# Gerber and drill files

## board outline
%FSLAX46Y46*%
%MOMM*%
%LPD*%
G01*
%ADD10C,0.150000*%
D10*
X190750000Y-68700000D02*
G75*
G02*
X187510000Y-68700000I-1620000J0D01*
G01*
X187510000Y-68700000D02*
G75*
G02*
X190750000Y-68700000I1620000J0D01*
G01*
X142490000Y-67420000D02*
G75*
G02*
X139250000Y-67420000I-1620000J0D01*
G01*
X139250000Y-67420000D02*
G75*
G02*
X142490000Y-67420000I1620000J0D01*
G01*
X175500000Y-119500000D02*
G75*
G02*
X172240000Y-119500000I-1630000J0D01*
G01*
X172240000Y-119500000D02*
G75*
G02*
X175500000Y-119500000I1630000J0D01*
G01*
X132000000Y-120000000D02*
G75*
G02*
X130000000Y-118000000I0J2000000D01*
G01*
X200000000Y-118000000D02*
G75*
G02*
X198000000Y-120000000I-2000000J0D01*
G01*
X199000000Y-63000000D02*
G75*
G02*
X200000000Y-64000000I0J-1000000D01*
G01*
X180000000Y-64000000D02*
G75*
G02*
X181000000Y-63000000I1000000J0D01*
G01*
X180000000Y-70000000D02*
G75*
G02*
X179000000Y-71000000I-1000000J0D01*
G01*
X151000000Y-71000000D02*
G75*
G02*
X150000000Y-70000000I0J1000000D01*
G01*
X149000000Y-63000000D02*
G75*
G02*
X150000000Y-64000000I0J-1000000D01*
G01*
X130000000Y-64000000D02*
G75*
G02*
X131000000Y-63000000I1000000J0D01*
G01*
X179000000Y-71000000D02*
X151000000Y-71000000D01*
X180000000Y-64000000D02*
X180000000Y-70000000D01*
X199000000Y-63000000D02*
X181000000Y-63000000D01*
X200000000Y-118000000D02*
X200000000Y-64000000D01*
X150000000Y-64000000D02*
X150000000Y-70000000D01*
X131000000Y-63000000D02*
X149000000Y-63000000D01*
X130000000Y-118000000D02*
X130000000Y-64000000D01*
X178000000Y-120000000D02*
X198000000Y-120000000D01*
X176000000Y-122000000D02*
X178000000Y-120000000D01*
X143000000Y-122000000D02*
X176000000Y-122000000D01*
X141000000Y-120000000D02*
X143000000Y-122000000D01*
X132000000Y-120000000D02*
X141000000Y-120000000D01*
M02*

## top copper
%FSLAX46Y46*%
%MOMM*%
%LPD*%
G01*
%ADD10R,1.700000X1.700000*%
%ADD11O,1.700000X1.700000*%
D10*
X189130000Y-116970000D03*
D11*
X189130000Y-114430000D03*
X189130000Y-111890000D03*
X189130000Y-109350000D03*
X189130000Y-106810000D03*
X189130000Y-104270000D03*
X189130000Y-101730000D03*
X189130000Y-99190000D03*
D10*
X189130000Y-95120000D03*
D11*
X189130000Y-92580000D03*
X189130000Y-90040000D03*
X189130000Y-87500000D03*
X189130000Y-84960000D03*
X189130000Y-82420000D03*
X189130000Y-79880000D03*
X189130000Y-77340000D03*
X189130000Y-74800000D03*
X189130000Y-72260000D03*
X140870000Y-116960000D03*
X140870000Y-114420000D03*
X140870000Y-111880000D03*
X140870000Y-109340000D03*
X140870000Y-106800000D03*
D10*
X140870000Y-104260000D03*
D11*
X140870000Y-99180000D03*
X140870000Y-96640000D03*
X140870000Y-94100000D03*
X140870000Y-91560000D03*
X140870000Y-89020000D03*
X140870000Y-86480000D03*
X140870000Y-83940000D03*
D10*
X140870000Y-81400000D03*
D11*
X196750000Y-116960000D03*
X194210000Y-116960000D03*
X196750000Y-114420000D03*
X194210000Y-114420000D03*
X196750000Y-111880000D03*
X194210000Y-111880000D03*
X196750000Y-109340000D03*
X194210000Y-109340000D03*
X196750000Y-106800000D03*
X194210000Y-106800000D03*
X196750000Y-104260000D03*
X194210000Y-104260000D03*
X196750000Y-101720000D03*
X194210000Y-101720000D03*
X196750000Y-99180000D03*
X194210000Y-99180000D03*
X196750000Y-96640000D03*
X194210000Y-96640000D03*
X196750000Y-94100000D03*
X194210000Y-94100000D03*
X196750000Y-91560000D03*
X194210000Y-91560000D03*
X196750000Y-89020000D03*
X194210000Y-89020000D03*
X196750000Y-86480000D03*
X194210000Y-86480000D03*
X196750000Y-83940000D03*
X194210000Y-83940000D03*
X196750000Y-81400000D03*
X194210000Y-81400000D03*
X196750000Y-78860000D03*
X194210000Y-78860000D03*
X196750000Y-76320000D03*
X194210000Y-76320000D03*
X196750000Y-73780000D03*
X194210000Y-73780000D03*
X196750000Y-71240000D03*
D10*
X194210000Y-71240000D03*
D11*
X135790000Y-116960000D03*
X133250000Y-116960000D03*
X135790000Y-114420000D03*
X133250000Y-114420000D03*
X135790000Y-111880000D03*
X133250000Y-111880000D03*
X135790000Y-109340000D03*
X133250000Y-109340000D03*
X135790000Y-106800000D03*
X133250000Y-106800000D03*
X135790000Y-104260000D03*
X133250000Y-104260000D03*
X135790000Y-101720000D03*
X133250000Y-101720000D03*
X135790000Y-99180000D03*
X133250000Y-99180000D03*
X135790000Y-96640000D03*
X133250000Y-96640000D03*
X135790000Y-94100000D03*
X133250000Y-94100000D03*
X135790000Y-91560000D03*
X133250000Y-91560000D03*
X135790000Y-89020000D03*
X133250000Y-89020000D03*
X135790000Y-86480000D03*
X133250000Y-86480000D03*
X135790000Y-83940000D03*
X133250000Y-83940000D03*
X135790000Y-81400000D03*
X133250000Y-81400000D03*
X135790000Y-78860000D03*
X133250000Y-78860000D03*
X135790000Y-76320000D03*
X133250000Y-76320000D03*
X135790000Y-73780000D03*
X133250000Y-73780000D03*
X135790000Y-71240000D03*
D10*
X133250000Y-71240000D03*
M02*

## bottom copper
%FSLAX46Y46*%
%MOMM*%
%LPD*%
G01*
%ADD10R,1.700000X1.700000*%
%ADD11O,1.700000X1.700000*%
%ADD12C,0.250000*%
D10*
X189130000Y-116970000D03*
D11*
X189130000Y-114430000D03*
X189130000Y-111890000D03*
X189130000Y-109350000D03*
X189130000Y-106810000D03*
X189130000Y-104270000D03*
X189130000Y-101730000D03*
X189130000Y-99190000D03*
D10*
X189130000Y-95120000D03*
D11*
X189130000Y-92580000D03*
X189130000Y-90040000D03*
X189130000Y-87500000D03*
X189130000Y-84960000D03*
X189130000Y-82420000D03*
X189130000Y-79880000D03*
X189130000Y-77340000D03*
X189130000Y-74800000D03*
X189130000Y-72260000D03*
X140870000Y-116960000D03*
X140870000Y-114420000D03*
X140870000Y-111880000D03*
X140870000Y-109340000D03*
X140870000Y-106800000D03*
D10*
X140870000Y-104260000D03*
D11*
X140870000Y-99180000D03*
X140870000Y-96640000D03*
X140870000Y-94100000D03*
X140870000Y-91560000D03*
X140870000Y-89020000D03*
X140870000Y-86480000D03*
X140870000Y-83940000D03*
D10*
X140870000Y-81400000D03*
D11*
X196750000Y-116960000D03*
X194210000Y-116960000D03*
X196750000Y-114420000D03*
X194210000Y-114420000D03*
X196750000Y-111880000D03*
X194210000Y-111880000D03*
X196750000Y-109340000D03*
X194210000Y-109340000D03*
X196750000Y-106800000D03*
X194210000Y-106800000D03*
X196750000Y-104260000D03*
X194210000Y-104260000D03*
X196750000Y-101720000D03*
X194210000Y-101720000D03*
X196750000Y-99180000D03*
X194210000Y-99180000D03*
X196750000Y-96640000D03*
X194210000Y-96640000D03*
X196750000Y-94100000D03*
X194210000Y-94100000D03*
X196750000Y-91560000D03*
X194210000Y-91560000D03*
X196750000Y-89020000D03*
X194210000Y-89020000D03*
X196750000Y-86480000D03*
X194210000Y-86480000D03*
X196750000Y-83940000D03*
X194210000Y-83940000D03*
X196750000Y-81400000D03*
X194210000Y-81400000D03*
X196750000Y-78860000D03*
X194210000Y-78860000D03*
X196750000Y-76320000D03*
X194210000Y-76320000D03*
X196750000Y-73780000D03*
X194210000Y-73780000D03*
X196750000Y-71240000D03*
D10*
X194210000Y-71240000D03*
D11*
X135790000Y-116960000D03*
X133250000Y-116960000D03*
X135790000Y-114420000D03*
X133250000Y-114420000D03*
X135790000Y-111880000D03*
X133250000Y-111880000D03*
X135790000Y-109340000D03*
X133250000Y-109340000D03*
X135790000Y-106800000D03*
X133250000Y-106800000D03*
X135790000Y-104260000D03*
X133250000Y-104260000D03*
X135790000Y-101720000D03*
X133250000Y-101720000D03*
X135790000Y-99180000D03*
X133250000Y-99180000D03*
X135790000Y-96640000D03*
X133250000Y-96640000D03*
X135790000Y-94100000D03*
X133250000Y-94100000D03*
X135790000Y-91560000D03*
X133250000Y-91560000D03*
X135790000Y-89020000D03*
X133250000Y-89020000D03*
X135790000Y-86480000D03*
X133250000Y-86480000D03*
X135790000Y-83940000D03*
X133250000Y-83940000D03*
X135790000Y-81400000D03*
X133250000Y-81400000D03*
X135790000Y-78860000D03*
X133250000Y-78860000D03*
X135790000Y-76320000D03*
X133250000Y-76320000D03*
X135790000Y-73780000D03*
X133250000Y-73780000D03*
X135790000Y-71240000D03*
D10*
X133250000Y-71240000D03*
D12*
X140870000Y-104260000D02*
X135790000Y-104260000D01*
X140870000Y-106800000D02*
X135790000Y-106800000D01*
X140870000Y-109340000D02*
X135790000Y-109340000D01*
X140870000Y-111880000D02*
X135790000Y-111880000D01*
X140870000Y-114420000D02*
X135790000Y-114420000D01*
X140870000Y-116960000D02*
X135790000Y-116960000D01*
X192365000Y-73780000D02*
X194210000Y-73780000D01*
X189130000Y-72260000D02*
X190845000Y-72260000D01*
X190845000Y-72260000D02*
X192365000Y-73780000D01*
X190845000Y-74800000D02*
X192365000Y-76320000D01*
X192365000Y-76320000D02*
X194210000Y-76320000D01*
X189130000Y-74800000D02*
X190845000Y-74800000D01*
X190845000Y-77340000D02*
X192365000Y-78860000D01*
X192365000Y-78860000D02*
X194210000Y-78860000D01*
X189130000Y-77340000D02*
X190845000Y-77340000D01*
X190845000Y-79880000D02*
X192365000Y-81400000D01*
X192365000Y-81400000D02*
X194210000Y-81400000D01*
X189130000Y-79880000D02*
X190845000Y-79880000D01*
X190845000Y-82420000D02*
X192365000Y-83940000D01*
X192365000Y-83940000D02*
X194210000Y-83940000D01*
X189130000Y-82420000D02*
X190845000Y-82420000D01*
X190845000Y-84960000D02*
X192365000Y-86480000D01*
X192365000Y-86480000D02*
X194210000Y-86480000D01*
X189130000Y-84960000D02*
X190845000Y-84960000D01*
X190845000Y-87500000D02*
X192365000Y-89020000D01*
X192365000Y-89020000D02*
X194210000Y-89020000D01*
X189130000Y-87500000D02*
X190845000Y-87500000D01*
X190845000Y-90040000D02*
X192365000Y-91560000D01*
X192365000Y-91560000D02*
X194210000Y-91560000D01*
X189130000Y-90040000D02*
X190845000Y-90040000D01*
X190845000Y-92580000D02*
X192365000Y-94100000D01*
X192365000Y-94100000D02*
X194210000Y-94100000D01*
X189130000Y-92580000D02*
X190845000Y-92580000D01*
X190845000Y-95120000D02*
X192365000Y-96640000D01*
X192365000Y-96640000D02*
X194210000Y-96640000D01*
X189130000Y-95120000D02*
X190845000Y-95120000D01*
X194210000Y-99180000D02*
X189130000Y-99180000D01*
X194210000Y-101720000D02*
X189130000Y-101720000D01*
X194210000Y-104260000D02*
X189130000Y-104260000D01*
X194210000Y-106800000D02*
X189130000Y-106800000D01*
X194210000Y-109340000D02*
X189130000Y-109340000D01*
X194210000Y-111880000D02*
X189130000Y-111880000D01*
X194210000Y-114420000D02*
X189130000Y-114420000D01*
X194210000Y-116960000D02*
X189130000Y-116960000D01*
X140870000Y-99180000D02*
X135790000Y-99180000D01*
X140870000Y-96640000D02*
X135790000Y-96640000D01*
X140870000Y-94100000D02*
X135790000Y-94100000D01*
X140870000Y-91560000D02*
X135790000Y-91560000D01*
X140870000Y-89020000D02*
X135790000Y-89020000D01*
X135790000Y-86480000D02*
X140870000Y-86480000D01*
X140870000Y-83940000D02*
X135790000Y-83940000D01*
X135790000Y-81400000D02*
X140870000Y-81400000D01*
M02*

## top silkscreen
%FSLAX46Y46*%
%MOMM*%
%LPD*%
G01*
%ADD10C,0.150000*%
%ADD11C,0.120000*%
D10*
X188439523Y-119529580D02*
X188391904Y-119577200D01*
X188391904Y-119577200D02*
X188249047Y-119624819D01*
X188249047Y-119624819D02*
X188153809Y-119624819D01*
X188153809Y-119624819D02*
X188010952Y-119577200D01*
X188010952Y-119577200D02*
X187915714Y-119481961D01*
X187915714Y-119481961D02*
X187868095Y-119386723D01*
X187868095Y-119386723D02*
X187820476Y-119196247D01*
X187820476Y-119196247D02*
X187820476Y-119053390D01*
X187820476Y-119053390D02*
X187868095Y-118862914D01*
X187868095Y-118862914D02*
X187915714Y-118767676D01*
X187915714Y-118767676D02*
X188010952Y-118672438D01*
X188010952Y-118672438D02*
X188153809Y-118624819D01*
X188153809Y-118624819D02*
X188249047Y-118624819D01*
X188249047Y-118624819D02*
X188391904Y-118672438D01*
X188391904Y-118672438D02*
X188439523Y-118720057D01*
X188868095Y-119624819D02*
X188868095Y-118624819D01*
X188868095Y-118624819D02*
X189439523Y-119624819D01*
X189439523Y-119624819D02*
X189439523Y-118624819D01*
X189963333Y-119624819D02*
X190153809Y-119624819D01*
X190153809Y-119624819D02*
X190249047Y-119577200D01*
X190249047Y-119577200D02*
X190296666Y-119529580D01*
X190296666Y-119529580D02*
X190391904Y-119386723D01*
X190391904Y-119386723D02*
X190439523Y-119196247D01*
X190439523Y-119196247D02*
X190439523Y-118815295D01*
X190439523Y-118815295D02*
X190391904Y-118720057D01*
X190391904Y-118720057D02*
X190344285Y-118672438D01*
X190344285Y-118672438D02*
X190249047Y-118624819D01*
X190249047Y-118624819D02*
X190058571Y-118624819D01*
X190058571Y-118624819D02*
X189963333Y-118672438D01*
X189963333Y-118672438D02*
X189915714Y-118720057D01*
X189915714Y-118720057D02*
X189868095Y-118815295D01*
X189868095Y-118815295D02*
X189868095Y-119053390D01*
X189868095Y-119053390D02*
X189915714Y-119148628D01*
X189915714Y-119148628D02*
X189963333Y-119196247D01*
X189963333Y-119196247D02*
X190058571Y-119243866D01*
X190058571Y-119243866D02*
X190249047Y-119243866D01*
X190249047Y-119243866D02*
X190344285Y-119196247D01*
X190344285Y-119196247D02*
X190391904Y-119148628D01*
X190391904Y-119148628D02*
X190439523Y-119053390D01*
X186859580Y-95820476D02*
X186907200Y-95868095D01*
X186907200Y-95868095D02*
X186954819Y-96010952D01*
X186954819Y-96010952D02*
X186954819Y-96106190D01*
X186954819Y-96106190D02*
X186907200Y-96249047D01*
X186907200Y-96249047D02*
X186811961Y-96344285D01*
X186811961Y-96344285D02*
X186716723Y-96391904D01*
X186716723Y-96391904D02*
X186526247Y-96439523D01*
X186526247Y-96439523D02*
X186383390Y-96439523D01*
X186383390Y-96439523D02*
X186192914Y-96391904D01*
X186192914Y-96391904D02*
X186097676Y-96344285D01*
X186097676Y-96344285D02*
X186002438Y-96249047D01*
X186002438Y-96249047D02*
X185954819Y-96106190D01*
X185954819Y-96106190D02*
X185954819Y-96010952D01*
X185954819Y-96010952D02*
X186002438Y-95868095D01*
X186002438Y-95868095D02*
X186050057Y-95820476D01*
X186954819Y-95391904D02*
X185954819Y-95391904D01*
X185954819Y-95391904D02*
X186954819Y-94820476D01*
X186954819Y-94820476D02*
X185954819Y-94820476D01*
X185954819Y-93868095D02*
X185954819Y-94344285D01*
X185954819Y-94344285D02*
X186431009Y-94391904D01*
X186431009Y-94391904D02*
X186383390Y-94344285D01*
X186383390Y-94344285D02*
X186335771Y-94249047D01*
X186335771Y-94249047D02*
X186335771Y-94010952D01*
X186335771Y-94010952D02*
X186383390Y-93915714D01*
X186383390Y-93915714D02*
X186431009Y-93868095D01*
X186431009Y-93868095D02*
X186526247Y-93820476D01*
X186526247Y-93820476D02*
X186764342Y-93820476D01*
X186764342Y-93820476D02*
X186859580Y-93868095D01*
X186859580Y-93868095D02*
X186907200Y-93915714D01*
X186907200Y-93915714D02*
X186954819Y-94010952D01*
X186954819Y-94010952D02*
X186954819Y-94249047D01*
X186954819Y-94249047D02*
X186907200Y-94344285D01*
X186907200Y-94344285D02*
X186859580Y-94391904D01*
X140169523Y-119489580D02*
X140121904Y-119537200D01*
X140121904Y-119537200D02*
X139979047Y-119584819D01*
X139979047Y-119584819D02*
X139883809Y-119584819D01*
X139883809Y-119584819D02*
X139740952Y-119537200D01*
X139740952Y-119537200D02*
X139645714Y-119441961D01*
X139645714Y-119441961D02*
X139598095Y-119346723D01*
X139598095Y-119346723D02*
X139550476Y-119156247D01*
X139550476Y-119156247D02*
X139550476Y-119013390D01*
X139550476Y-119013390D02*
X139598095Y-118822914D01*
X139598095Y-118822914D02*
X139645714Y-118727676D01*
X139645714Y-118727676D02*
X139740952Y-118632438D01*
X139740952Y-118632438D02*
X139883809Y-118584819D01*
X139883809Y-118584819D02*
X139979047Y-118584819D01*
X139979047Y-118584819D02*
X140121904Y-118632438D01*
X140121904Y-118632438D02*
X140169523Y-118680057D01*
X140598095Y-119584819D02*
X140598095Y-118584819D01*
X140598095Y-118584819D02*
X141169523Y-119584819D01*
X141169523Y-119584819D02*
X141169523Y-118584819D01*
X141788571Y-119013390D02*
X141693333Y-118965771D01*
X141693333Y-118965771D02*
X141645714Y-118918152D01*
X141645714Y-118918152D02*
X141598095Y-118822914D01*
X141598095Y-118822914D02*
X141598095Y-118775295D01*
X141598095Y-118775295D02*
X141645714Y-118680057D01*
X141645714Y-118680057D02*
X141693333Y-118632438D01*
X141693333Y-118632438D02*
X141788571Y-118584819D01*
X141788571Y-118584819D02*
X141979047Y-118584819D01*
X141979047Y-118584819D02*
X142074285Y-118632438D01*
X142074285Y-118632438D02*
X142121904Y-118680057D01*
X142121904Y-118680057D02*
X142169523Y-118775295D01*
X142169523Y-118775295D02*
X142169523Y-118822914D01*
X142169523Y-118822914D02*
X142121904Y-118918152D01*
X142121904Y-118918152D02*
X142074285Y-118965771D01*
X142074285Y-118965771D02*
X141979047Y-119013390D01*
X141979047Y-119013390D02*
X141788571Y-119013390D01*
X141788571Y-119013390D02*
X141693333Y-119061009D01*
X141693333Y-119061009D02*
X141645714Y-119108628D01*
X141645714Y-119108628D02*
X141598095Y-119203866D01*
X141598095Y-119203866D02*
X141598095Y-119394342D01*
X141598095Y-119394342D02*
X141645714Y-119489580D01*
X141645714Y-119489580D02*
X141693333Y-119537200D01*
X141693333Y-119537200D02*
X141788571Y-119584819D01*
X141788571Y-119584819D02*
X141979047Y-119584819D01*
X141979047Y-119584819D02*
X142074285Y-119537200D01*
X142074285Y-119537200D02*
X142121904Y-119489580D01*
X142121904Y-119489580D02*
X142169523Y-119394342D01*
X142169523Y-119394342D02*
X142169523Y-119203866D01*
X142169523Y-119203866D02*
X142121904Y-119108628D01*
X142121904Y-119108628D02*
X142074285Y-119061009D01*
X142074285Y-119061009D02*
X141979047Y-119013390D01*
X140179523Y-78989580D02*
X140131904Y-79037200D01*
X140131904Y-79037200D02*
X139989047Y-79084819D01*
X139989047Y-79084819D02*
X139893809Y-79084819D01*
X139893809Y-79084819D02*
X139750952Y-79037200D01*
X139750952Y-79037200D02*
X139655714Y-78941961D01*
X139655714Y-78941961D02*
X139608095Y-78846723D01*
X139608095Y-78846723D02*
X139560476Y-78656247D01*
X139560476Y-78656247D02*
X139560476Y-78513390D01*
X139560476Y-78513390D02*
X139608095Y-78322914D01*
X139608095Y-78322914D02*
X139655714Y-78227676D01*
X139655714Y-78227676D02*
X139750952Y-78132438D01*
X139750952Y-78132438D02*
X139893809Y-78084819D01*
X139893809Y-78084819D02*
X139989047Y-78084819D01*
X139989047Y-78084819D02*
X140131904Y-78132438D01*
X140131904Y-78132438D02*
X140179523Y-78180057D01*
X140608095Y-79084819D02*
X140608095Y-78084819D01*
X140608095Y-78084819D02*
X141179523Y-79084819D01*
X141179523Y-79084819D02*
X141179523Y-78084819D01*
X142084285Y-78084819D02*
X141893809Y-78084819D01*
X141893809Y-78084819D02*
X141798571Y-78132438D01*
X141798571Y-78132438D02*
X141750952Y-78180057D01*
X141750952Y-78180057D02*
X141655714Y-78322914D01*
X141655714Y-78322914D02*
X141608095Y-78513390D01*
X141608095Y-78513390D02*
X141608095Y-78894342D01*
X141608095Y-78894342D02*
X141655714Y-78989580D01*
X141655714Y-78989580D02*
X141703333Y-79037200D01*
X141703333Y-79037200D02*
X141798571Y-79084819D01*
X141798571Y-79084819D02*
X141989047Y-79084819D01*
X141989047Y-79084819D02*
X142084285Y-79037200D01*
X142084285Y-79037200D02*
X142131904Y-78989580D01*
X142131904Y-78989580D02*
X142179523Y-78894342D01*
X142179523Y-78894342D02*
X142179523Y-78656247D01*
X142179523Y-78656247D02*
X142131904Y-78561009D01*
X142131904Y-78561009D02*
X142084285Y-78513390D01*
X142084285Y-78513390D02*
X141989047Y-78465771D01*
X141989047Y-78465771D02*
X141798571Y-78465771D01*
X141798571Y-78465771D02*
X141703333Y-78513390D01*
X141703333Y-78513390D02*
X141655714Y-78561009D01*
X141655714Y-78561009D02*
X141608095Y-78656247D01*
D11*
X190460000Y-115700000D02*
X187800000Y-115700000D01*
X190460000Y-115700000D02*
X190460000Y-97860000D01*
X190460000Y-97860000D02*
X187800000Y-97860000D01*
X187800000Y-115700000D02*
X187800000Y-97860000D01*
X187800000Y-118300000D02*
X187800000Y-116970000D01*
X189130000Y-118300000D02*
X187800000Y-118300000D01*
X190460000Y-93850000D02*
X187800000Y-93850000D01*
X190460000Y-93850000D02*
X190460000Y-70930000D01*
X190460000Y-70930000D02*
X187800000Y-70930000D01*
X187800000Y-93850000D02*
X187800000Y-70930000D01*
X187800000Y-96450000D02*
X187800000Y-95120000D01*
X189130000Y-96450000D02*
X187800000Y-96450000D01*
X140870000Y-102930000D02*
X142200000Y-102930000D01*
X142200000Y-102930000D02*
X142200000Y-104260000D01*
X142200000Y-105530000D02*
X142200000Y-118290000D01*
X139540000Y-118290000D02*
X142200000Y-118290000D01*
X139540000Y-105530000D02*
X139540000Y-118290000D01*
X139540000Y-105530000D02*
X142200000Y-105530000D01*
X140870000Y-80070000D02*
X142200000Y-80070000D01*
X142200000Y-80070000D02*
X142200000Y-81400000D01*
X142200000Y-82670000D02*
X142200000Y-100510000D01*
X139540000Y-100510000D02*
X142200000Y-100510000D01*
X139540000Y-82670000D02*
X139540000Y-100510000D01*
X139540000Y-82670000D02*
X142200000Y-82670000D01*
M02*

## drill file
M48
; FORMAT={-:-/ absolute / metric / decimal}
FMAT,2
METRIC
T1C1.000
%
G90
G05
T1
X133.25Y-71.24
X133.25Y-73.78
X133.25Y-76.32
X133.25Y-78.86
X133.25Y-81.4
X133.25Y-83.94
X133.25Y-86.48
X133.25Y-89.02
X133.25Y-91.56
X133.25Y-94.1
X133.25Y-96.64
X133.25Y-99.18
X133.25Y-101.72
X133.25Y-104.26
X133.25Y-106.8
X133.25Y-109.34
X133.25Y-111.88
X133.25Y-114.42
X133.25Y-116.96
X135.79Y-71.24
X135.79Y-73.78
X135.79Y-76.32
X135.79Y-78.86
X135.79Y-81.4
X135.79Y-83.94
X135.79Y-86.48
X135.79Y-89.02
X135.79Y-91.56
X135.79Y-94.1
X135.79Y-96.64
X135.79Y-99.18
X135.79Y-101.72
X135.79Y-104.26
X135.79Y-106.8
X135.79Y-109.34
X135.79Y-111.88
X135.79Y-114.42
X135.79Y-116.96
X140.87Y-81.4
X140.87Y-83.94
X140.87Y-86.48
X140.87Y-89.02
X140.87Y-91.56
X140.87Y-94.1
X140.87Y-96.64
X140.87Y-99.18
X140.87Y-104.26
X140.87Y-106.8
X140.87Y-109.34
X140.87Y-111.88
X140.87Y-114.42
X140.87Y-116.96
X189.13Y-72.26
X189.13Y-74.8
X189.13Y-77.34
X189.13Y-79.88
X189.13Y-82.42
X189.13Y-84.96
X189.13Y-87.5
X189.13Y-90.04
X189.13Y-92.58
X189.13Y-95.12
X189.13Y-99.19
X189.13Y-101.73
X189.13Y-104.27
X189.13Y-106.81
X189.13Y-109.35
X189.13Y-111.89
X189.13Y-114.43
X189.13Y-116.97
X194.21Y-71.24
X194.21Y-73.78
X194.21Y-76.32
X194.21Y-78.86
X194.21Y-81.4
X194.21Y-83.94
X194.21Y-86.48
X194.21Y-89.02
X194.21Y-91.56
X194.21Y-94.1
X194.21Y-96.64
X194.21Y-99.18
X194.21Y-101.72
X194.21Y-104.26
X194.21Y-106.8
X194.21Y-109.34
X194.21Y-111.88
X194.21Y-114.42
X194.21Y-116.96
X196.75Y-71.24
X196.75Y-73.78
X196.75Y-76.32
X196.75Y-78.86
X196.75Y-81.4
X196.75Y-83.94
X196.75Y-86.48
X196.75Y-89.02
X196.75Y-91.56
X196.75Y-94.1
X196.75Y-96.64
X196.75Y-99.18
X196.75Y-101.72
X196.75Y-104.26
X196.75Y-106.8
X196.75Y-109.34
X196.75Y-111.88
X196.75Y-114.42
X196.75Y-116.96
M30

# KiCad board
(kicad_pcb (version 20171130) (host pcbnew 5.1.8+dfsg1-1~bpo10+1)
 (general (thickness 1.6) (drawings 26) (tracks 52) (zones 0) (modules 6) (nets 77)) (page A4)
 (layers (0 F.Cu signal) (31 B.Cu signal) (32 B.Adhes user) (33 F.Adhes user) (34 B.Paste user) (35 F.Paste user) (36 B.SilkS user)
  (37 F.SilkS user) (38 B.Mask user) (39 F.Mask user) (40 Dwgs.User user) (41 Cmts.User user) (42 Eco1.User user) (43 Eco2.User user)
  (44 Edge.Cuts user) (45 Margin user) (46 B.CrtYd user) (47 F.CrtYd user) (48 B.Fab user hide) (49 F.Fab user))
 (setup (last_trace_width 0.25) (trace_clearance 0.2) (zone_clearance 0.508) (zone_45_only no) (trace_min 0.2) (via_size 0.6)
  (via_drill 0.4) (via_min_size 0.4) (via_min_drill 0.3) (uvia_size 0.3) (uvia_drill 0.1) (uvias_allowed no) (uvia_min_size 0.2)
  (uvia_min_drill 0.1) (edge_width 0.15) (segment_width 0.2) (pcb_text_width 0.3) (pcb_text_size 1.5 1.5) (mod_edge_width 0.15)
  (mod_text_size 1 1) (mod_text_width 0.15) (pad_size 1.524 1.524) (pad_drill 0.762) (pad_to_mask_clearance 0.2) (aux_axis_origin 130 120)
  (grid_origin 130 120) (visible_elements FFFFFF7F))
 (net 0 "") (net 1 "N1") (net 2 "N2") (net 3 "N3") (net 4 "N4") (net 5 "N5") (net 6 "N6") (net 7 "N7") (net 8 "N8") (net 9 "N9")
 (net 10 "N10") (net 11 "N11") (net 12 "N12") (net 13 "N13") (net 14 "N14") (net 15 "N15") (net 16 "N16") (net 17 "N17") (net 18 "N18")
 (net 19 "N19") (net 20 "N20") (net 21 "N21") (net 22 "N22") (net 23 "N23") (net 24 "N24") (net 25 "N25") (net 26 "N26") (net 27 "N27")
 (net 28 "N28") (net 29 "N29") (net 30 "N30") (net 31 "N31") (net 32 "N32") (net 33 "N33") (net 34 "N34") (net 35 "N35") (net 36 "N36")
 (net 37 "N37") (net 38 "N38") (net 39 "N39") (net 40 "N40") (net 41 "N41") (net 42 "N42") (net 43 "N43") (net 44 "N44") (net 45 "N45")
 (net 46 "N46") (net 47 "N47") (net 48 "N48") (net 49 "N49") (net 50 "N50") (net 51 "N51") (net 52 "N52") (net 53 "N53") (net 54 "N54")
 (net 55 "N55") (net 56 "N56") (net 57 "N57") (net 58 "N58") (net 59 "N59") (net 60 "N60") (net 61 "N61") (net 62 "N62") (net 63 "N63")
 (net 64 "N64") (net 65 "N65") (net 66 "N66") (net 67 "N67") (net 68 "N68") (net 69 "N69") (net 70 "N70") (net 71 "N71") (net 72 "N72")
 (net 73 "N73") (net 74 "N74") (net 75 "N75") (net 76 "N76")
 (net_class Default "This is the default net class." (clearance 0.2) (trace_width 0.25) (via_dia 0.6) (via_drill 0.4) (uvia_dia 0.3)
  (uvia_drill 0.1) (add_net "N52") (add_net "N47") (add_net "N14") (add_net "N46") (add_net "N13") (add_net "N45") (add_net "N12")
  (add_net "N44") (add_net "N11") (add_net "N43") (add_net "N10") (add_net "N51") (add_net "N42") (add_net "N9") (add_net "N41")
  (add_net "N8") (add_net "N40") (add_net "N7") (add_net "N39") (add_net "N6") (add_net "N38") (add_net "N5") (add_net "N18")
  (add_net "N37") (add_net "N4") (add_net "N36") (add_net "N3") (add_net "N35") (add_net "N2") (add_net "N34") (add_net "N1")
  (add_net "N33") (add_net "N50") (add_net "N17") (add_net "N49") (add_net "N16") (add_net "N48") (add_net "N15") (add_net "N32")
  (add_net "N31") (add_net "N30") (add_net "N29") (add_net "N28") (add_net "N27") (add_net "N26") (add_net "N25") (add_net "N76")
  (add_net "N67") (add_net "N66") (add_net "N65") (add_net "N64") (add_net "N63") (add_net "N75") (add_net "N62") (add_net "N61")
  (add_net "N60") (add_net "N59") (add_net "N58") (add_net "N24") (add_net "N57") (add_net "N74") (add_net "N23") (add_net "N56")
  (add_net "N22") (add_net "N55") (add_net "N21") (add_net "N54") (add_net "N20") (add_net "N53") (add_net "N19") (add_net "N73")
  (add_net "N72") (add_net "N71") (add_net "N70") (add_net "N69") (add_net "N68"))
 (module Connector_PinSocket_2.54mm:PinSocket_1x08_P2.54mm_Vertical (layer F.Cu) (at 189.13 116.97 180)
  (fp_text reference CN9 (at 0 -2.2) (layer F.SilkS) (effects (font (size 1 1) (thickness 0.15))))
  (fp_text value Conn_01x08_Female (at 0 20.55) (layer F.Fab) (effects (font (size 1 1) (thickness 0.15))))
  (fp_line (start -1.33 1.27) (end 1.33 1.27) (layer F.SilkS) (width 0.12))
  (fp_line (start -1.33 1.27) (end -1.33 19.11) (layer F.SilkS) (width 0.12))
  (fp_line (start -1.33 19.11) (end 1.33 19.11) (layer F.SilkS) (width 0.12))
  (fp_line (start 1.33 1.27) (end 1.33 19.11) (layer F.SilkS) (width 0.12))
  (fp_line (start 1.33 -1.33) (end 1.33 0) (layer F.SilkS) (width 0.12))
  (fp_line (start 0 -1.33) (end 1.33 -1.33) (layer F.SilkS) (width 0.12))
  (pad 1 thru_hole rect (at 0 0 180) (size 1.7 1.7) (drill 1) (layers *.Cu *.Mask) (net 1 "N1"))
  (pad 2 thru_hole oval (at 0 2.54 180) (size 1.7 1.7) (drill 1) (layers *.Cu *.Mask) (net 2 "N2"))
  (pad 3 thru_hole oval (at 0 5.08 180) (size 1.7 1.7) (drill 1) (layers *.Cu *.Mask) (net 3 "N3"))
  (pad 4 thru_hole oval (at 0 7.62 180) (size 1.7 1.7) (drill 1) (layers *.Cu *.Mask) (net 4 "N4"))
  (pad 5 thru_hole oval (at 0 10.16 180) (size 1.7 1.7) (drill 1) (layers *.Cu *.Mask) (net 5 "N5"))
  (pad 6 thru_hole oval (at 0 12.7 180) (size 1.7 1.7) (drill 1) (layers *.Cu *.Mask) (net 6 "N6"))
  (pad 7 thru_hole oval (at 0 15.24 180) (size 1.7 1.7) (drill 1) (layers *.Cu *.Mask) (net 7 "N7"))
  (pad 8 thru_hole oval (at 0 17.78 180) (size 1.7 1.7) (drill 1) (layers *.Cu *.Mask) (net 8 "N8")))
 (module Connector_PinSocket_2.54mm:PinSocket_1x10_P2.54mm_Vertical (layer F.Cu) (at 189.13 95.12 180)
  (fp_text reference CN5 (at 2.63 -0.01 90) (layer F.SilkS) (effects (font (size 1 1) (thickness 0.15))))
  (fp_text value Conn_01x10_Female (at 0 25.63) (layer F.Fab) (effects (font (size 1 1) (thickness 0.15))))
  (fp_line (start -1.33 1.27) (end 1.33 1.27) (layer F.SilkS) (width 0.12))
  (fp_line (start -1.33 1.27) (end -1.33 24.19) (layer F.SilkS) (width 0.12))
  (fp_line (start -1.33 24.19) (end 1.33 24.19) (layer F.SilkS) (width 0.12))
  (fp_line (start 1.33 1.27) (end 1.33 24.19) (layer F.SilkS) (width 0.12))
  (fp_line (start 1.33 -1.33) (end 1.33 0) (layer F.SilkS) (width 0.12))
  (fp_line (start 0 -1.33) (end 1.33 -1.33) (layer F.SilkS) (width 0.12))
  (pad 1 thru_hole rect (at 0 0 180) (size 1.7 1.7) (drill 1) (layers *.Cu *.Mask) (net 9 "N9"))
  (pad 2 thru_hole oval (at 0 2.54 180) (size 1.7 1.7) (drill 1) (layers *.Cu *.Mask) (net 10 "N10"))
  (pad 3 thru_hole oval (at 0 5.08 180) (size 1.7 1.7) (drill 1) (layers *.Cu *.Mask) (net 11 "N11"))
  (pad 4 thru_hole oval (at 0 7.62 180) (size 1.7 1.7) (drill 1) (layers *.Cu *.Mask) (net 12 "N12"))
  (pad 5 thru_hole oval (at 0 10.16 180) (size 1.7 1.7) (drill 1) (layers *.Cu *.Mask) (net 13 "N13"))
  (pad 6 thru_hole oval (at 0 12.7 180) (size 1.7 1.7) (drill 1) (layers *.Cu *.Mask) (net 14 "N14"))
  (pad 7 thru_hole oval (at 0 15.24 180) (size 1.7 1.7) (drill 1) (layers *.Cu *.Mask) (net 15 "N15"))
  (pad 8 thru_hole oval (at 0 17.78 180) (size 1.7 1.7) (drill 1) (layers *.Cu *.Mask) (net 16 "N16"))
  (pad 9 thru_hole oval (at 0 20.32 180) (size 1.7 1.7) (drill 1) (layers *.Cu *.Mask) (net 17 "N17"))
  (pad 10 thru_hole oval (at 0 22.86 180) (size 1.7 1.7) (drill 1) (layers *.Cu *.Mask) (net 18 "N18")))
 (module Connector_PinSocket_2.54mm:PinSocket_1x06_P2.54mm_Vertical (layer F.Cu) (at 140.87 104.26)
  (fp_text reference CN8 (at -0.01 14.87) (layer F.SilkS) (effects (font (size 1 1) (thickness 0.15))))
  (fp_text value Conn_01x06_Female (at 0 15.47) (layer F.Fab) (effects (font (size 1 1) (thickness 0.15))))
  (fp_line (start 0 -1.33) (end 1.33 -1.33) (layer F.SilkS) (width 0.12))
  (fp_line (start 1.33 -1.33) (end 1.33 0) (layer F.SilkS) (width 0.12))
  (fp_line (start 1.33 1.27) (end 1.33 14.03) (layer F.SilkS) (width 0.12))
  (fp_line (start -1.33 14.03) (end 1.33 14.03) (layer F.SilkS) (width 0.12))
  (fp_line (start -1.33 1.27) (end -1.33 14.03) (layer F.SilkS) (width 0.12))
  (fp_line (start -1.33 1.27) (end 1.33 1.27) (layer F.SilkS) (width 0.12))
  (pad 6 thru_hole oval (at 0 12.7) (size 1.7 1.7) (drill 1) (layers *.Cu *.Mask) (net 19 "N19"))
  (pad 5 thru_hole oval (at 0 10.16) (size 1.7 1.7) (drill 1) (layers *.Cu *.Mask) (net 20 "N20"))
  (pad 4 thru_hole oval (at 0 7.62) (size 1.7 1.7) (drill 1) (layers *.Cu *.Mask) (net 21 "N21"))
  (pad 3 thru_hole oval (at 0 5.08) (size 1.7 1.7) (drill 1) (layers *.Cu *.Mask) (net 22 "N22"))
  (pad 2 thru_hole oval (at 0 2.54) (size 1.7 1.7) (drill 1) (layers *.Cu *.Mask) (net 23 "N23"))
  (pad 1 thru_hole rect (at 0 0) (size 1.7 1.7) (drill 1) (layers *.Cu *.Mask) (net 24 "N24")))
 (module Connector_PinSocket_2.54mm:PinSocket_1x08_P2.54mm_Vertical (layer F.Cu) (at 140.87 81.4)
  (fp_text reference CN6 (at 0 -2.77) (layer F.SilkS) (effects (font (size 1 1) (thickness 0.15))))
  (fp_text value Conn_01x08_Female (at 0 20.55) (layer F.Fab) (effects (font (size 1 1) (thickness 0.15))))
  (fp_line (start 0 -1.33) (end 1.33 -1.33) (layer F.SilkS) (width 0.12))
  (fp_line (start 1.33 -1.33) (end 1.33 0) (layer F.SilkS) (width 0.12))
  (fp_line (start 1.33 1.27) (end 1.33 19.11) (layer F.SilkS) (width 0.12))
  (fp_line (start -1.33 19.11) (end 1.33 19.11) (layer F.SilkS) (width 0.12))
  (fp_line (start -1.33 1.27) (end -1.33 19.11) (layer F.SilkS) (width 0.12))
  (fp_line (start -1.33 1.27) (end 1.33 1.27) (layer F.SilkS) (width 0.12))
  (pad 8 thru_hole oval (at 0 17.78) (size 1.7 1.7) (drill 1) (layers *.Cu *.Mask) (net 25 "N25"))
  (pad 7 thru_hole oval (at 0 15.24) (size 1.7 1.7) (drill 1) (layers *.Cu *.Mask) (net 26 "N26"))
  (pad 6 thru_hole oval (at 0 12.7) (size 1.7 1.7) (drill 1) (layers *.Cu *.Mask) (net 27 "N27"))
  (pad 5 thru_hole oval (at 0 10.16) (size 1.7 1.7) (drill 1) (layers *.Cu *.Mask) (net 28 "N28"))
  (pad 4 thru_hole oval (at 0 7.62) (size 1.7 1.7) (drill 1) (layers *.Cu *.Mask) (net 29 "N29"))
  (pad 3 thru_hole oval (at 0 5.08) (size 1.7 1.7) (drill 1) (layers *.Cu *.Mask) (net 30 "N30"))
  (pad 2 thru_hole oval (at 0 2.54) (size 1.7 1.7) (drill 1) (layers *.Cu *.Mask) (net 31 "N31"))
  (pad 1 thru_hole rect (at 0 0) (size 1.7 1.7) (drill 1) (layers *.Cu *.Mask) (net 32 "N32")))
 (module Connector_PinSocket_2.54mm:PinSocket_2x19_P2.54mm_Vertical (layer B.Cu) (at 194.21 71.24 180)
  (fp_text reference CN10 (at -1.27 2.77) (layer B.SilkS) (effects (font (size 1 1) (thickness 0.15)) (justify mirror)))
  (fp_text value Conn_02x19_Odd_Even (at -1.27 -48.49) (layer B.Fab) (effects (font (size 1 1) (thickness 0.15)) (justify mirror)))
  (pad 38 thru_hole oval (at -2.54 -45.72 180) (size 1.7 1.7) (drill 1) (layers *.Cu *.Mask) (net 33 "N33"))
  (pad 37 thru_hole oval (at 0 -45.72 180) (size 1.7 1.7) (drill 1) (layers *.Cu *.Mask) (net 1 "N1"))
  (pad 36 thru_hole oval (at -2.54 -43.18 180) (size 1.7 1.7) (drill 1) (layers *.Cu *.Mask) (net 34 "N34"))
  (pad 35 thru_hole oval (at 0 -43.18 180) (size 1.7 1.7) (drill 1) (layers *.Cu *.Mask) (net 2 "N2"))
  (pad 34 thru_hole oval (at -2.54 -40.64 180) (size 1.7 1.7) (drill 1) (layers *.Cu *.Mask) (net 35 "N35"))
  (pad 33 thru_hole oval (at 0 -40.64 180) (size 1.7 1.7) (drill 1) (layers *.Cu *.Mask) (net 3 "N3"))
  (pad 32 thru_hole oval (at -2.54 -38.1 180) (size 1.7 1.7) (drill 1) (layers *.Cu *.Mask) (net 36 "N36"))
  (pad 31 thru_hole oval (at 0 -38.1 180) (size 1.7 1.7) (drill 1) (layers *.Cu *.Mask) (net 4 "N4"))
  (pad 30 thru_hole oval (at -2.54 -35.56 180) (size 1.7 1.7) (drill 1) (layers *.Cu *.Mask) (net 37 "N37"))
  (pad 29 thru_hole oval (at 0 -35.56 180) (size 1.7 1.7) (drill 1) (layers *.Cu *.Mask) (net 5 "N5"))
  (pad 28 thru_hole oval (at -2.54 -33.02 180) (size 1.7 1.7) (drill 1) (layers *.Cu *.Mask) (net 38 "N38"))
  (pad 27 thru_hole oval (at 0 -33.02 180) (size 1.7 1.7) (drill 1) (layers *.Cu *.Mask) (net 6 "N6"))
  (pad 26 thru_hole oval (at -2.54 -30.48 180) (size 1.7 1.7) (drill 1) (layers *.Cu *.Mask) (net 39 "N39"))
  (pad 25 thru_hole oval (at 0 -30.48 180) (size 1.7 1.7) (drill 1) (layers *.Cu *.Mask) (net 7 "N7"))
  (pad 24 thru_hole oval (at -2.54 -27.94 180) (size 1.7 1.7) (drill 1) (layers *.Cu *.Mask) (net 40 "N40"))
  (pad 23 thru_hole oval (at 0 -27.94 180) (size 1.7 1.7) (drill 1) (layers *.Cu *.Mask) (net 8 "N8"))
  (pad 22 thru_hole oval (at -2.54 -25.4 180) (size 1.7 1.7) (drill 1) (layers *.Cu *.Mask) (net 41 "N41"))
  (pad 21 thru_hole oval (at 0 -25.4 180) (size 1.7 1.7) (drill 1) (layers *.Cu *.Mask) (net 9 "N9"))
  (pad 20 thru_hole oval (at -2.54 -22.86 180) (size 1.7 1.7) (drill 1) (layers *.Cu *.Mask) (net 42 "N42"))
  (pad 19 thru_hole oval (at 0 -22.86 180) (size 1.7 1.7) (drill 1) (layers *.Cu *.Mask) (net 10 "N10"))
  (pad 18 thru_hole oval (at -2.54 -20.32 180) (size 1.7 1.7) (drill 1) (layers *.Cu *.Mask) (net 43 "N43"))
  (pad 17 thru_hole oval (at 0 -20.32 180) (size 1.7 1.7) (drill 1) (layers *.Cu *.Mask) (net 11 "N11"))
  (pad 16 thru_hole oval (at -2.54 -17.78 180) (size 1.7 1.7) (drill 1) (layers *.Cu *.Mask) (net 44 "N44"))
  (pad 15 thru_hole oval (at 0 -17.78 180) (size 1.7 1.7) (drill 1) (layers *.Cu *.Mask) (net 12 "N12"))
  (pad 14 thru_hole oval (at -2.54 -15.24 180) (size 1.7 1.7) (drill 1) (layers *.Cu *.Mask) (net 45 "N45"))
  (pad 13 thru_hole oval (at 0 -15.24 180) (size 1.7 1.7) (drill 1) (layers *.Cu *.Mask) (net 13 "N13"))
  (pad 12 thru_hole oval (at -2.54 -12.7 180) (size 1.7 1.7) (drill 1) (layers *.Cu *.Mask) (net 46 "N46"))
  (pad 11 thru_hole oval (at 0 -12.7 180) (size 1.7 1.7) (drill 1) (layers *.Cu *.Mask) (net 14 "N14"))
  (pad 10 thru_hole oval (at -2.54 -10.16 180) (size 1.7 1.7) (drill 1) (layers *.Cu *.Mask) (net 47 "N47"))
  (pad 9 thru_hole oval (at 0 -10.16 180) (size 1.7 1.7) (drill 1) (layers *.Cu *.Mask) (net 15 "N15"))
  (pad 8 thru_hole oval (at -2.54 -7.62 180) (size 1.7 1.7) (drill 1) (layers *.Cu *.Mask) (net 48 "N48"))
  (pad 7 thru_hole oval (at 0 -7.62 180) (size 1.7 1.7) (drill 1) (layers *.Cu *.Mask) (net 16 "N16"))
  (pad 6 thru_hole oval (at -2.54 -5.08 180) (size 1.7 1.7) (drill 1) (layers *.Cu *.Mask) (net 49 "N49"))
  (pad 5 thru_hole oval (at 0 -5.08 180) (size 1.7 1.7) (drill 1) (layers *.Cu *.Mask) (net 17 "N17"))
  (pad 4 thru_hole oval (at -2.54 -2.54 180) (size 1.7 1.7) (drill 1) (layers *.Cu *.Mask) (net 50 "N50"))
  (pad 3 thru_hole oval (at 0 -2.54 180) (size 1.7 1.7) (drill 1) (layers *.Cu *.Mask) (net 18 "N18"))
  (pad 2 thru_hole oval (at -2.54 0 180) (size 1.7 1.7) (drill 1) (layers *.Cu *.Mask) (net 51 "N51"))
  (pad 1 thru_hole rect (at 0 0 180) (size 1.7 1.7) (drill 1) (layers *.Cu *.Mask) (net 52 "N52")))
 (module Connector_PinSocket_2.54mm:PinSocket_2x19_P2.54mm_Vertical (layer B.Cu) (at 133.25 71.24 180)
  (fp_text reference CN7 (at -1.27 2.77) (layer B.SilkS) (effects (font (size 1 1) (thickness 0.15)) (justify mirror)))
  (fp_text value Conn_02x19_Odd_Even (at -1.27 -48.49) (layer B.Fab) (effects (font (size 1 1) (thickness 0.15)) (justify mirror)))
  (pad 38 thru_hole oval (at -2.54 -45.72 180) (size 1.7 1.7) (drill 1) (layers *.Cu *.Mask) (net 19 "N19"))
  (pad 37 thru_hole oval (at 0 -45.72 180) (size 1.7 1.7) (drill 1) (layers *.Cu *.Mask) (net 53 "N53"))
  (pad 36 thru_hole oval (at -2.54 -43.18 180) (size 1.7 1.7) (drill 1) (layers *.Cu *.Mask) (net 20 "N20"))
  (pad 35 thru_hole oval (at 0 -43.18 180) (size 1.7 1.7) (drill 1) (layers *.Cu *.Mask) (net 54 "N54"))
  (pad 34 thru_hole oval (at -2.54 -40.64 180) (size 1.7 1.7) (drill 1) (layers *.Cu *.Mask) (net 21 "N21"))
  (pad 33 thru_hole oval (at 0 -40.64 180) (size 1.7 1.7) (drill 1) (layers *.Cu *.Mask) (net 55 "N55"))
  (pad 32 thru_hole oval (at -2.54 -38.1 180) (size 1.7 1.7) (drill 1) (layers *.Cu *.Mask) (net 22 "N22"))
  (pad 31 thru_hole oval (at 0 -38.1 180) (size 1.7 1.7) (drill 1) (layers *.Cu *.Mask) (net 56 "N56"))
  (pad 30 thru_hole oval (at -2.54 -35.56 180) (size 1.7 1.7) (drill 1) (layers *.Cu *.Mask) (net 23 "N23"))
  (pad 29 thru_hole oval (at 0 -35.56 180) (size 1.7 1.7) (drill 1) (layers *.Cu *.Mask) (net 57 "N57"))
  (pad 28 thru_hole oval (at -2.54 -33.02 180) (size 1.7 1.7) (drill 1) (layers *.Cu *.Mask) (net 24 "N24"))
  (pad 27 thru_hole oval (at 0 -33.02 180) (size 1.7 1.7) (drill 1) (layers *.Cu *.Mask) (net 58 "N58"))
  (pad 26 thru_hole oval (at -2.54 -30.48 180) (size 1.7 1.7) (drill 1) (layers *.Cu *.Mask) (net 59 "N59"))
  (pad 25 thru_hole oval (at 0 -30.48 180) (size 1.7 1.7) (drill 1) (layers *.Cu *.Mask) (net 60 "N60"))
  (pad 24 thru_hole oval (at -2.54 -27.94 180) (size 1.7 1.7) (drill 1) (layers *.Cu *.Mask) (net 25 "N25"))
  (pad 23 thru_hole oval (at 0 -27.94 180) (size 1.7 1.7) (drill 1) (layers *.Cu *.Mask) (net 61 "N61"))
  (pad 22 thru_hole oval (at -2.54 -25.4 180) (size 1.7 1.7) (drill 1) (layers *.Cu *.Mask) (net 26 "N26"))
  (pad 21 thru_hole oval (at 0 -25.4 180) (size 1.7 1.7) (drill 1) (layers *.Cu *.Mask) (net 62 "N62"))
  (pad 20 thru_hole oval (at -2.54 -22.86 180) (size 1.7 1.7) (drill 1) (layers *.Cu *.Mask) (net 27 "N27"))
  (pad 19 thru_hole oval (at 0 -22.86 180) (size 1.7 1.7) (drill 1) (layers *.Cu *.Mask) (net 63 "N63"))
  (pad 18 thru_hole oval (at -2.54 -20.32 180) (size 1.7 1.7) (drill 1) (layers *.Cu *.Mask) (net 28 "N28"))
  (pad 17 thru_hole oval (at 0 -20.32 180) (size 1.7 1.7) (drill 1) (layers *.Cu *.Mask) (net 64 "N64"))
  (pad 16 thru_hole oval (at -2.54 -17.78 180) (size 1.7 1.7) (drill 1) (layers *.Cu *.Mask) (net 29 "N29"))
  (pad 15 thru_hole oval (at 0 -17.78 180) (size 1.7 1.7) (drill 1) (layers *.Cu *.Mask) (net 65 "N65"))
  (pad 14 thru_hole oval (at -2.54 -15.24 180) (size 1.7 1.7) (drill 1) (layers *.Cu *.Mask) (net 30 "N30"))
  (pad 13 thru_hole oval (at 0 -15.24 180) (size 1.7 1.7) (drill 1) (layers *.Cu *.Mask) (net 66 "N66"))
  (pad 12 thru_hole oval (at -2.54 -12.7 180) (size 1.7 1.7) (drill 1) (layers *.Cu *.Mask) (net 31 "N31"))
  (pad 11 thru_hole oval (at 0 -12.7 180) (size 1.7 1.7) (drill 1) (layers *.Cu *.Mask) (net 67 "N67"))
  (pad 10 thru_hole oval (at -2.54 -10.16 180) (size 1.7 1.7) (drill 1) (layers *.Cu *.Mask) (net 32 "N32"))
  (pad 9 thru_hole oval (at 0 -10.16 180) (size 1.7 1.7) (drill 1) (layers *.Cu *.Mask) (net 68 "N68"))
  (pad 8 thru_hole oval (at -2.54 -7.62 180) (size 1.7 1.7) (drill 1) (layers *.Cu *.Mask) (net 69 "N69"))
  (pad 7 thru_hole oval (at 0 -7.62 180) (size 1.7 1.7) (drill 1) (layers *.Cu *.Mask) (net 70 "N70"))
  (pad 6 thru_hole oval (at -2.54 -5.08 180) (size 1.7 1.7) (drill 1) (layers *.Cu *.Mask) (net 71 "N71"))
  (pad 5 thru_hole oval (at 0 -5.08 180) (size 1.7 1.7) (drill 1) (layers *.Cu *.Mask) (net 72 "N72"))
  (pad 4 thru_hole oval (at -2.54 -2.54 180) (size 1.7 1.7) (drill 1) (layers *.Cu *.Mask) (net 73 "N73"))
  (pad 3 thru_hole oval (at 0 -2.54 180) (size 1.7 1.7) (drill 1) (layers *.Cu *.Mask) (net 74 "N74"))
  (pad 2 thru_hole oval (at -2.54 0 180) (size 1.7 1.7) (drill 1) (layers *.Cu *.Mask) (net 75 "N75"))
  (pad 1 thru_hole rect (at 0 0 180) (size 1.7 1.7) (drill 1) (layers *.Cu *.Mask) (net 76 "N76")))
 (gr_circle (center 189.13 68.7) (end 190.75 68.7) (layer Edge.Cuts) (width 0.15))
 (gr_circle (center 140.87 67.42) (end 142.49 67.42) (layer Edge.Cuts) (width 0.15))
 (gr_circle (center 173.87 119.5) (end 175.5 119.5) (layer Edge.Cuts) (width 0.15))
 (gr_arc (start 132 118) (end 132 120) (angle 90) (layer Edge.Cuts) (width 0.15))
 (gr_arc (start 198 118) (end 200 118) (angle 90) (layer Edge.Cuts) (width 0.15))
 (gr_arc (start 199 64) (end 199 63) (angle 90) (layer Edge.Cuts) (width 0.15))
 (gr_arc (start 181 64) (end 180 64) (angle 90) (layer Edge.Cuts) (width 0.15))
 (gr_arc (start 179 70) (end 180 70) (angle 90) (layer Edge.Cuts) (width 0.15))
 (gr_arc (start 151 70) (end 151 71) (angle 90) (layer Edge.Cuts) (width 0.15))
 (gr_arc (start 149 64) (end 149 63) (angle 90) (layer Edge.Cuts) (width 0.15))
 (gr_arc (start 131 64) (end 130 64) (angle 90) (layer Edge.Cuts) (width 0.15))
 (gr_line (start 179 71) (end 151 71) (layer Edge.Cuts) (width 0.15))
 (gr_line (start 180 64) (end 180 70) (layer Edge.Cuts) (width 0.15))
 (gr_line (start 199 63) (end 181 63) (layer Edge.Cuts) (width 0.15))
 (gr_line (start 200 118) (end 200 64) (layer Edge.Cuts) (width 0.15))
 (gr_line (start 150 64) (end 150 70) (layer Edge.Cuts) (width 0.15))
 (gr_line (start 131 63) (end 149 63) (layer Edge.Cuts) (width 0.15))
 (gr_line (start 130 118) (end 130 64) (layer Edge.Cuts) (width 0.15))
 (gr_line (start 178 120) (end 198 120) (layer Edge.Cuts) (width 0.15))
 (gr_line (start 176 122) (end 178 120) (layer Edge.Cuts) (width 0.15))
 (gr_line (start 143 122) (end 176 122) (layer Edge.Cuts) (width 0.15))
 (gr_line (start 141 120) (end 143 122) (layer Edge.Cuts) (width 0.15))
 (gr_line (start 132 120) (end 141 120) (layer Edge.Cuts) (width 0.15))
 (segment (start 140.87 104.26) (end 135.79 104.26) (width 0.25) (layer B.Cu) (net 24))
 (segment (start 140.87 106.8) (end 135.79 106.8) (width 0.25) (layer B.Cu) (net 23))
 (segment (start 140.87 109.34) (end 135.79 109.34) (width 0.25) (layer B.Cu) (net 22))
 (segment (start 140.87 111.88) (end 135.79 111.88) (width 0.25) (layer B.Cu) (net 21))
 (segment (start 140.87 114.42) (end 135.79 114.42) (width 0.25) (layer B.Cu) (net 20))
 (segment (start 140.87 116.96) (end 135.79 116.96) (width 0.25) (layer B.Cu) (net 19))
 (segment (start 192.365 73.78) (end 194.21 73.78) (width 0.25) (layer B.Cu) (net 18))
 (segment (start 189.13 72.26) (end 190.845 72.26) (width 0.25) (layer B.Cu) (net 18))
 (segment (start 190.845 72.26) (end 192.365 73.78) (width 0.25) (layer B.Cu) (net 18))
 (segment (start 190.845 74.8) (end 192.365 76.32) (width 0.25) (layer B.Cu) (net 17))
 (segment (start 192.365 76.32) (end 194.21 76.32) (width 0.25) (layer B.Cu) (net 17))
 (segment (start 189.13 74.8) (end 190.845 74.8) (width 0.25) (layer B.Cu) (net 17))
 (segment (start 190.845 77.34) (end 192.365 78.86) (width 0.25) (layer B.Cu) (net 16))
 (segment (start 192.365 78.86) (end 194.21 78.86) (width 0.25) (layer B.Cu) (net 16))
 (segment (start 189.13 77.34) (end 190.845 77.34) (width 0.25) (layer B.Cu) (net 16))
 (segment (start 190.845 79.88) (end 192.365 81.4) (width 0.25) (layer B.Cu) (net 15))
 (segment (start 192.365 81.4) (end 194.21 81.4) (width 0.25) (layer B.Cu) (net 15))
 (segment (start 189.13 79.88) (end 190.845 79.88) (width 0.25) (layer B.Cu) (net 15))
 (segment (start 190.845 82.42) (end 192.365 83.94) (width 0.25) (layer B.Cu) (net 14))
 (segment (start 192.365 83.94) (end 194.21 83.94) (width 0.25) (layer B.Cu) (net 14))
 (segment (start 189.13 82.42) (end 190.845 82.42) (width 0.25) (layer B.Cu) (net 14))
 (segment (start 190.845 84.96) (end 192.365 86.48) (width 0.25) (layer B.Cu) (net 13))
 (segment (start 192.365 86.48) (end 194.21 86.48) (width 0.25) (layer B.Cu) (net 13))
 (segment (start 189.13 84.96) (end 190.845 84.96) (width 0.25) (layer B.Cu) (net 13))
 (segment (start 190.845 87.5) (end 192.365 89.02) (width 0.25) (layer B.Cu) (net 12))
 (segment (start 192.365 89.02) (end 194.21 89.02) (width 0.25) (layer B.Cu) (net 12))
 (segment (start 189.13 87.5) (end 190.845 87.5) (width 0.25) (layer B.Cu) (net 12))
 (segment (start 190.845 90.04) (end 192.365 91.56) (width 0.25) (layer B.Cu) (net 11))
 (segment (start 192.365 91.56) (end 194.21 91.56) (width 0.25) (layer B.Cu) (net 11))
 (segment (start 189.13 90.04) (end 190.845 90.04) (width 0.25) (layer B.Cu) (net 11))
 (segment (start 190.845 92.58) (end 192.365 94.1) (width 0.25) (layer B.Cu) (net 10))
 (segment (start 192.365 94.1) (end 194.21 94.1) (width 0.25) (layer B.Cu) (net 10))
 (segment (start 189.13 92.58) (end 190.845 92.58) (width 0.25) (layer B.Cu) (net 10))
 (segment (start 190.845 95.12) (end 192.365 96.64) (width 0.25) (layer B.Cu) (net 9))
 (segment (start 192.365 96.64) (end 194.21 96.64) (width 0.25) (layer B.Cu) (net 9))
 (segment (start 189.13 95.12) (end 190.845 95.12) (width 0.25) (layer B.Cu) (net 9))
 (segment (start 194.21 99.18) (end 189.13 99.18) (width 0.25) (layer B.Cu) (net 8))
 (segment (start 194.21 101.72) (end 189.13 101.72) (width 0.25) (layer B.Cu) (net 7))
 (segment (start 194.21 104.26) (end 189.13 104.26) (width 0.25) (layer B.Cu) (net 6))
 (segment (start 194.21 106.8) (end 189.13 106.8) (width 0.25) (layer B.Cu) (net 5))
 (segment (start 194.21 109.34) (end 189.13 109.34) (width 0.25) (layer B.Cu) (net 4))
 (segment (start 194.21 111.88) (end 189.13 111.88) (width 0.25) (layer B.Cu) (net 3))
 (segment (start 194.21 114.42) (end 189.13 114.42) (width 0.25) (layer B.Cu) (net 2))
 (segment (start 194.21 116.96) (end 189.13 116.96) (width 0.25) (layer B.Cu) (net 1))
 (segment (start 140.87 99.18) (end 135.79 99.18) (width 0.25) (layer B.Cu) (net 25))
 (segment (start 140.87 96.64) (end 135.79 96.64) (width 0.25) (layer B.Cu) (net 26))
 (segment (start 140.87 94.1) (end 135.79 94.1) (width 0.25) (layer B.Cu) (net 27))
 (segment (start 140.87 91.56) (end 135.79 91.56) (width 0.25) (layer B.Cu) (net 28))
 (segment (start 140.87 89.02) (end 135.79 89.02) (width 0.25) (layer B.Cu) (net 29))
 (segment (start 135.79 86.48) (end 140.87 86.48) (width 0.25) (layer B.Cu) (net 30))
 (segment (start 140.87 83.94) (end 135.79 83.94) (width 0.25) (layer B.Cu) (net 31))
 (segment (start 135.79 81.4) (end 140.87 81.4) (width 0.25) (layer B.Cu) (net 32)))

